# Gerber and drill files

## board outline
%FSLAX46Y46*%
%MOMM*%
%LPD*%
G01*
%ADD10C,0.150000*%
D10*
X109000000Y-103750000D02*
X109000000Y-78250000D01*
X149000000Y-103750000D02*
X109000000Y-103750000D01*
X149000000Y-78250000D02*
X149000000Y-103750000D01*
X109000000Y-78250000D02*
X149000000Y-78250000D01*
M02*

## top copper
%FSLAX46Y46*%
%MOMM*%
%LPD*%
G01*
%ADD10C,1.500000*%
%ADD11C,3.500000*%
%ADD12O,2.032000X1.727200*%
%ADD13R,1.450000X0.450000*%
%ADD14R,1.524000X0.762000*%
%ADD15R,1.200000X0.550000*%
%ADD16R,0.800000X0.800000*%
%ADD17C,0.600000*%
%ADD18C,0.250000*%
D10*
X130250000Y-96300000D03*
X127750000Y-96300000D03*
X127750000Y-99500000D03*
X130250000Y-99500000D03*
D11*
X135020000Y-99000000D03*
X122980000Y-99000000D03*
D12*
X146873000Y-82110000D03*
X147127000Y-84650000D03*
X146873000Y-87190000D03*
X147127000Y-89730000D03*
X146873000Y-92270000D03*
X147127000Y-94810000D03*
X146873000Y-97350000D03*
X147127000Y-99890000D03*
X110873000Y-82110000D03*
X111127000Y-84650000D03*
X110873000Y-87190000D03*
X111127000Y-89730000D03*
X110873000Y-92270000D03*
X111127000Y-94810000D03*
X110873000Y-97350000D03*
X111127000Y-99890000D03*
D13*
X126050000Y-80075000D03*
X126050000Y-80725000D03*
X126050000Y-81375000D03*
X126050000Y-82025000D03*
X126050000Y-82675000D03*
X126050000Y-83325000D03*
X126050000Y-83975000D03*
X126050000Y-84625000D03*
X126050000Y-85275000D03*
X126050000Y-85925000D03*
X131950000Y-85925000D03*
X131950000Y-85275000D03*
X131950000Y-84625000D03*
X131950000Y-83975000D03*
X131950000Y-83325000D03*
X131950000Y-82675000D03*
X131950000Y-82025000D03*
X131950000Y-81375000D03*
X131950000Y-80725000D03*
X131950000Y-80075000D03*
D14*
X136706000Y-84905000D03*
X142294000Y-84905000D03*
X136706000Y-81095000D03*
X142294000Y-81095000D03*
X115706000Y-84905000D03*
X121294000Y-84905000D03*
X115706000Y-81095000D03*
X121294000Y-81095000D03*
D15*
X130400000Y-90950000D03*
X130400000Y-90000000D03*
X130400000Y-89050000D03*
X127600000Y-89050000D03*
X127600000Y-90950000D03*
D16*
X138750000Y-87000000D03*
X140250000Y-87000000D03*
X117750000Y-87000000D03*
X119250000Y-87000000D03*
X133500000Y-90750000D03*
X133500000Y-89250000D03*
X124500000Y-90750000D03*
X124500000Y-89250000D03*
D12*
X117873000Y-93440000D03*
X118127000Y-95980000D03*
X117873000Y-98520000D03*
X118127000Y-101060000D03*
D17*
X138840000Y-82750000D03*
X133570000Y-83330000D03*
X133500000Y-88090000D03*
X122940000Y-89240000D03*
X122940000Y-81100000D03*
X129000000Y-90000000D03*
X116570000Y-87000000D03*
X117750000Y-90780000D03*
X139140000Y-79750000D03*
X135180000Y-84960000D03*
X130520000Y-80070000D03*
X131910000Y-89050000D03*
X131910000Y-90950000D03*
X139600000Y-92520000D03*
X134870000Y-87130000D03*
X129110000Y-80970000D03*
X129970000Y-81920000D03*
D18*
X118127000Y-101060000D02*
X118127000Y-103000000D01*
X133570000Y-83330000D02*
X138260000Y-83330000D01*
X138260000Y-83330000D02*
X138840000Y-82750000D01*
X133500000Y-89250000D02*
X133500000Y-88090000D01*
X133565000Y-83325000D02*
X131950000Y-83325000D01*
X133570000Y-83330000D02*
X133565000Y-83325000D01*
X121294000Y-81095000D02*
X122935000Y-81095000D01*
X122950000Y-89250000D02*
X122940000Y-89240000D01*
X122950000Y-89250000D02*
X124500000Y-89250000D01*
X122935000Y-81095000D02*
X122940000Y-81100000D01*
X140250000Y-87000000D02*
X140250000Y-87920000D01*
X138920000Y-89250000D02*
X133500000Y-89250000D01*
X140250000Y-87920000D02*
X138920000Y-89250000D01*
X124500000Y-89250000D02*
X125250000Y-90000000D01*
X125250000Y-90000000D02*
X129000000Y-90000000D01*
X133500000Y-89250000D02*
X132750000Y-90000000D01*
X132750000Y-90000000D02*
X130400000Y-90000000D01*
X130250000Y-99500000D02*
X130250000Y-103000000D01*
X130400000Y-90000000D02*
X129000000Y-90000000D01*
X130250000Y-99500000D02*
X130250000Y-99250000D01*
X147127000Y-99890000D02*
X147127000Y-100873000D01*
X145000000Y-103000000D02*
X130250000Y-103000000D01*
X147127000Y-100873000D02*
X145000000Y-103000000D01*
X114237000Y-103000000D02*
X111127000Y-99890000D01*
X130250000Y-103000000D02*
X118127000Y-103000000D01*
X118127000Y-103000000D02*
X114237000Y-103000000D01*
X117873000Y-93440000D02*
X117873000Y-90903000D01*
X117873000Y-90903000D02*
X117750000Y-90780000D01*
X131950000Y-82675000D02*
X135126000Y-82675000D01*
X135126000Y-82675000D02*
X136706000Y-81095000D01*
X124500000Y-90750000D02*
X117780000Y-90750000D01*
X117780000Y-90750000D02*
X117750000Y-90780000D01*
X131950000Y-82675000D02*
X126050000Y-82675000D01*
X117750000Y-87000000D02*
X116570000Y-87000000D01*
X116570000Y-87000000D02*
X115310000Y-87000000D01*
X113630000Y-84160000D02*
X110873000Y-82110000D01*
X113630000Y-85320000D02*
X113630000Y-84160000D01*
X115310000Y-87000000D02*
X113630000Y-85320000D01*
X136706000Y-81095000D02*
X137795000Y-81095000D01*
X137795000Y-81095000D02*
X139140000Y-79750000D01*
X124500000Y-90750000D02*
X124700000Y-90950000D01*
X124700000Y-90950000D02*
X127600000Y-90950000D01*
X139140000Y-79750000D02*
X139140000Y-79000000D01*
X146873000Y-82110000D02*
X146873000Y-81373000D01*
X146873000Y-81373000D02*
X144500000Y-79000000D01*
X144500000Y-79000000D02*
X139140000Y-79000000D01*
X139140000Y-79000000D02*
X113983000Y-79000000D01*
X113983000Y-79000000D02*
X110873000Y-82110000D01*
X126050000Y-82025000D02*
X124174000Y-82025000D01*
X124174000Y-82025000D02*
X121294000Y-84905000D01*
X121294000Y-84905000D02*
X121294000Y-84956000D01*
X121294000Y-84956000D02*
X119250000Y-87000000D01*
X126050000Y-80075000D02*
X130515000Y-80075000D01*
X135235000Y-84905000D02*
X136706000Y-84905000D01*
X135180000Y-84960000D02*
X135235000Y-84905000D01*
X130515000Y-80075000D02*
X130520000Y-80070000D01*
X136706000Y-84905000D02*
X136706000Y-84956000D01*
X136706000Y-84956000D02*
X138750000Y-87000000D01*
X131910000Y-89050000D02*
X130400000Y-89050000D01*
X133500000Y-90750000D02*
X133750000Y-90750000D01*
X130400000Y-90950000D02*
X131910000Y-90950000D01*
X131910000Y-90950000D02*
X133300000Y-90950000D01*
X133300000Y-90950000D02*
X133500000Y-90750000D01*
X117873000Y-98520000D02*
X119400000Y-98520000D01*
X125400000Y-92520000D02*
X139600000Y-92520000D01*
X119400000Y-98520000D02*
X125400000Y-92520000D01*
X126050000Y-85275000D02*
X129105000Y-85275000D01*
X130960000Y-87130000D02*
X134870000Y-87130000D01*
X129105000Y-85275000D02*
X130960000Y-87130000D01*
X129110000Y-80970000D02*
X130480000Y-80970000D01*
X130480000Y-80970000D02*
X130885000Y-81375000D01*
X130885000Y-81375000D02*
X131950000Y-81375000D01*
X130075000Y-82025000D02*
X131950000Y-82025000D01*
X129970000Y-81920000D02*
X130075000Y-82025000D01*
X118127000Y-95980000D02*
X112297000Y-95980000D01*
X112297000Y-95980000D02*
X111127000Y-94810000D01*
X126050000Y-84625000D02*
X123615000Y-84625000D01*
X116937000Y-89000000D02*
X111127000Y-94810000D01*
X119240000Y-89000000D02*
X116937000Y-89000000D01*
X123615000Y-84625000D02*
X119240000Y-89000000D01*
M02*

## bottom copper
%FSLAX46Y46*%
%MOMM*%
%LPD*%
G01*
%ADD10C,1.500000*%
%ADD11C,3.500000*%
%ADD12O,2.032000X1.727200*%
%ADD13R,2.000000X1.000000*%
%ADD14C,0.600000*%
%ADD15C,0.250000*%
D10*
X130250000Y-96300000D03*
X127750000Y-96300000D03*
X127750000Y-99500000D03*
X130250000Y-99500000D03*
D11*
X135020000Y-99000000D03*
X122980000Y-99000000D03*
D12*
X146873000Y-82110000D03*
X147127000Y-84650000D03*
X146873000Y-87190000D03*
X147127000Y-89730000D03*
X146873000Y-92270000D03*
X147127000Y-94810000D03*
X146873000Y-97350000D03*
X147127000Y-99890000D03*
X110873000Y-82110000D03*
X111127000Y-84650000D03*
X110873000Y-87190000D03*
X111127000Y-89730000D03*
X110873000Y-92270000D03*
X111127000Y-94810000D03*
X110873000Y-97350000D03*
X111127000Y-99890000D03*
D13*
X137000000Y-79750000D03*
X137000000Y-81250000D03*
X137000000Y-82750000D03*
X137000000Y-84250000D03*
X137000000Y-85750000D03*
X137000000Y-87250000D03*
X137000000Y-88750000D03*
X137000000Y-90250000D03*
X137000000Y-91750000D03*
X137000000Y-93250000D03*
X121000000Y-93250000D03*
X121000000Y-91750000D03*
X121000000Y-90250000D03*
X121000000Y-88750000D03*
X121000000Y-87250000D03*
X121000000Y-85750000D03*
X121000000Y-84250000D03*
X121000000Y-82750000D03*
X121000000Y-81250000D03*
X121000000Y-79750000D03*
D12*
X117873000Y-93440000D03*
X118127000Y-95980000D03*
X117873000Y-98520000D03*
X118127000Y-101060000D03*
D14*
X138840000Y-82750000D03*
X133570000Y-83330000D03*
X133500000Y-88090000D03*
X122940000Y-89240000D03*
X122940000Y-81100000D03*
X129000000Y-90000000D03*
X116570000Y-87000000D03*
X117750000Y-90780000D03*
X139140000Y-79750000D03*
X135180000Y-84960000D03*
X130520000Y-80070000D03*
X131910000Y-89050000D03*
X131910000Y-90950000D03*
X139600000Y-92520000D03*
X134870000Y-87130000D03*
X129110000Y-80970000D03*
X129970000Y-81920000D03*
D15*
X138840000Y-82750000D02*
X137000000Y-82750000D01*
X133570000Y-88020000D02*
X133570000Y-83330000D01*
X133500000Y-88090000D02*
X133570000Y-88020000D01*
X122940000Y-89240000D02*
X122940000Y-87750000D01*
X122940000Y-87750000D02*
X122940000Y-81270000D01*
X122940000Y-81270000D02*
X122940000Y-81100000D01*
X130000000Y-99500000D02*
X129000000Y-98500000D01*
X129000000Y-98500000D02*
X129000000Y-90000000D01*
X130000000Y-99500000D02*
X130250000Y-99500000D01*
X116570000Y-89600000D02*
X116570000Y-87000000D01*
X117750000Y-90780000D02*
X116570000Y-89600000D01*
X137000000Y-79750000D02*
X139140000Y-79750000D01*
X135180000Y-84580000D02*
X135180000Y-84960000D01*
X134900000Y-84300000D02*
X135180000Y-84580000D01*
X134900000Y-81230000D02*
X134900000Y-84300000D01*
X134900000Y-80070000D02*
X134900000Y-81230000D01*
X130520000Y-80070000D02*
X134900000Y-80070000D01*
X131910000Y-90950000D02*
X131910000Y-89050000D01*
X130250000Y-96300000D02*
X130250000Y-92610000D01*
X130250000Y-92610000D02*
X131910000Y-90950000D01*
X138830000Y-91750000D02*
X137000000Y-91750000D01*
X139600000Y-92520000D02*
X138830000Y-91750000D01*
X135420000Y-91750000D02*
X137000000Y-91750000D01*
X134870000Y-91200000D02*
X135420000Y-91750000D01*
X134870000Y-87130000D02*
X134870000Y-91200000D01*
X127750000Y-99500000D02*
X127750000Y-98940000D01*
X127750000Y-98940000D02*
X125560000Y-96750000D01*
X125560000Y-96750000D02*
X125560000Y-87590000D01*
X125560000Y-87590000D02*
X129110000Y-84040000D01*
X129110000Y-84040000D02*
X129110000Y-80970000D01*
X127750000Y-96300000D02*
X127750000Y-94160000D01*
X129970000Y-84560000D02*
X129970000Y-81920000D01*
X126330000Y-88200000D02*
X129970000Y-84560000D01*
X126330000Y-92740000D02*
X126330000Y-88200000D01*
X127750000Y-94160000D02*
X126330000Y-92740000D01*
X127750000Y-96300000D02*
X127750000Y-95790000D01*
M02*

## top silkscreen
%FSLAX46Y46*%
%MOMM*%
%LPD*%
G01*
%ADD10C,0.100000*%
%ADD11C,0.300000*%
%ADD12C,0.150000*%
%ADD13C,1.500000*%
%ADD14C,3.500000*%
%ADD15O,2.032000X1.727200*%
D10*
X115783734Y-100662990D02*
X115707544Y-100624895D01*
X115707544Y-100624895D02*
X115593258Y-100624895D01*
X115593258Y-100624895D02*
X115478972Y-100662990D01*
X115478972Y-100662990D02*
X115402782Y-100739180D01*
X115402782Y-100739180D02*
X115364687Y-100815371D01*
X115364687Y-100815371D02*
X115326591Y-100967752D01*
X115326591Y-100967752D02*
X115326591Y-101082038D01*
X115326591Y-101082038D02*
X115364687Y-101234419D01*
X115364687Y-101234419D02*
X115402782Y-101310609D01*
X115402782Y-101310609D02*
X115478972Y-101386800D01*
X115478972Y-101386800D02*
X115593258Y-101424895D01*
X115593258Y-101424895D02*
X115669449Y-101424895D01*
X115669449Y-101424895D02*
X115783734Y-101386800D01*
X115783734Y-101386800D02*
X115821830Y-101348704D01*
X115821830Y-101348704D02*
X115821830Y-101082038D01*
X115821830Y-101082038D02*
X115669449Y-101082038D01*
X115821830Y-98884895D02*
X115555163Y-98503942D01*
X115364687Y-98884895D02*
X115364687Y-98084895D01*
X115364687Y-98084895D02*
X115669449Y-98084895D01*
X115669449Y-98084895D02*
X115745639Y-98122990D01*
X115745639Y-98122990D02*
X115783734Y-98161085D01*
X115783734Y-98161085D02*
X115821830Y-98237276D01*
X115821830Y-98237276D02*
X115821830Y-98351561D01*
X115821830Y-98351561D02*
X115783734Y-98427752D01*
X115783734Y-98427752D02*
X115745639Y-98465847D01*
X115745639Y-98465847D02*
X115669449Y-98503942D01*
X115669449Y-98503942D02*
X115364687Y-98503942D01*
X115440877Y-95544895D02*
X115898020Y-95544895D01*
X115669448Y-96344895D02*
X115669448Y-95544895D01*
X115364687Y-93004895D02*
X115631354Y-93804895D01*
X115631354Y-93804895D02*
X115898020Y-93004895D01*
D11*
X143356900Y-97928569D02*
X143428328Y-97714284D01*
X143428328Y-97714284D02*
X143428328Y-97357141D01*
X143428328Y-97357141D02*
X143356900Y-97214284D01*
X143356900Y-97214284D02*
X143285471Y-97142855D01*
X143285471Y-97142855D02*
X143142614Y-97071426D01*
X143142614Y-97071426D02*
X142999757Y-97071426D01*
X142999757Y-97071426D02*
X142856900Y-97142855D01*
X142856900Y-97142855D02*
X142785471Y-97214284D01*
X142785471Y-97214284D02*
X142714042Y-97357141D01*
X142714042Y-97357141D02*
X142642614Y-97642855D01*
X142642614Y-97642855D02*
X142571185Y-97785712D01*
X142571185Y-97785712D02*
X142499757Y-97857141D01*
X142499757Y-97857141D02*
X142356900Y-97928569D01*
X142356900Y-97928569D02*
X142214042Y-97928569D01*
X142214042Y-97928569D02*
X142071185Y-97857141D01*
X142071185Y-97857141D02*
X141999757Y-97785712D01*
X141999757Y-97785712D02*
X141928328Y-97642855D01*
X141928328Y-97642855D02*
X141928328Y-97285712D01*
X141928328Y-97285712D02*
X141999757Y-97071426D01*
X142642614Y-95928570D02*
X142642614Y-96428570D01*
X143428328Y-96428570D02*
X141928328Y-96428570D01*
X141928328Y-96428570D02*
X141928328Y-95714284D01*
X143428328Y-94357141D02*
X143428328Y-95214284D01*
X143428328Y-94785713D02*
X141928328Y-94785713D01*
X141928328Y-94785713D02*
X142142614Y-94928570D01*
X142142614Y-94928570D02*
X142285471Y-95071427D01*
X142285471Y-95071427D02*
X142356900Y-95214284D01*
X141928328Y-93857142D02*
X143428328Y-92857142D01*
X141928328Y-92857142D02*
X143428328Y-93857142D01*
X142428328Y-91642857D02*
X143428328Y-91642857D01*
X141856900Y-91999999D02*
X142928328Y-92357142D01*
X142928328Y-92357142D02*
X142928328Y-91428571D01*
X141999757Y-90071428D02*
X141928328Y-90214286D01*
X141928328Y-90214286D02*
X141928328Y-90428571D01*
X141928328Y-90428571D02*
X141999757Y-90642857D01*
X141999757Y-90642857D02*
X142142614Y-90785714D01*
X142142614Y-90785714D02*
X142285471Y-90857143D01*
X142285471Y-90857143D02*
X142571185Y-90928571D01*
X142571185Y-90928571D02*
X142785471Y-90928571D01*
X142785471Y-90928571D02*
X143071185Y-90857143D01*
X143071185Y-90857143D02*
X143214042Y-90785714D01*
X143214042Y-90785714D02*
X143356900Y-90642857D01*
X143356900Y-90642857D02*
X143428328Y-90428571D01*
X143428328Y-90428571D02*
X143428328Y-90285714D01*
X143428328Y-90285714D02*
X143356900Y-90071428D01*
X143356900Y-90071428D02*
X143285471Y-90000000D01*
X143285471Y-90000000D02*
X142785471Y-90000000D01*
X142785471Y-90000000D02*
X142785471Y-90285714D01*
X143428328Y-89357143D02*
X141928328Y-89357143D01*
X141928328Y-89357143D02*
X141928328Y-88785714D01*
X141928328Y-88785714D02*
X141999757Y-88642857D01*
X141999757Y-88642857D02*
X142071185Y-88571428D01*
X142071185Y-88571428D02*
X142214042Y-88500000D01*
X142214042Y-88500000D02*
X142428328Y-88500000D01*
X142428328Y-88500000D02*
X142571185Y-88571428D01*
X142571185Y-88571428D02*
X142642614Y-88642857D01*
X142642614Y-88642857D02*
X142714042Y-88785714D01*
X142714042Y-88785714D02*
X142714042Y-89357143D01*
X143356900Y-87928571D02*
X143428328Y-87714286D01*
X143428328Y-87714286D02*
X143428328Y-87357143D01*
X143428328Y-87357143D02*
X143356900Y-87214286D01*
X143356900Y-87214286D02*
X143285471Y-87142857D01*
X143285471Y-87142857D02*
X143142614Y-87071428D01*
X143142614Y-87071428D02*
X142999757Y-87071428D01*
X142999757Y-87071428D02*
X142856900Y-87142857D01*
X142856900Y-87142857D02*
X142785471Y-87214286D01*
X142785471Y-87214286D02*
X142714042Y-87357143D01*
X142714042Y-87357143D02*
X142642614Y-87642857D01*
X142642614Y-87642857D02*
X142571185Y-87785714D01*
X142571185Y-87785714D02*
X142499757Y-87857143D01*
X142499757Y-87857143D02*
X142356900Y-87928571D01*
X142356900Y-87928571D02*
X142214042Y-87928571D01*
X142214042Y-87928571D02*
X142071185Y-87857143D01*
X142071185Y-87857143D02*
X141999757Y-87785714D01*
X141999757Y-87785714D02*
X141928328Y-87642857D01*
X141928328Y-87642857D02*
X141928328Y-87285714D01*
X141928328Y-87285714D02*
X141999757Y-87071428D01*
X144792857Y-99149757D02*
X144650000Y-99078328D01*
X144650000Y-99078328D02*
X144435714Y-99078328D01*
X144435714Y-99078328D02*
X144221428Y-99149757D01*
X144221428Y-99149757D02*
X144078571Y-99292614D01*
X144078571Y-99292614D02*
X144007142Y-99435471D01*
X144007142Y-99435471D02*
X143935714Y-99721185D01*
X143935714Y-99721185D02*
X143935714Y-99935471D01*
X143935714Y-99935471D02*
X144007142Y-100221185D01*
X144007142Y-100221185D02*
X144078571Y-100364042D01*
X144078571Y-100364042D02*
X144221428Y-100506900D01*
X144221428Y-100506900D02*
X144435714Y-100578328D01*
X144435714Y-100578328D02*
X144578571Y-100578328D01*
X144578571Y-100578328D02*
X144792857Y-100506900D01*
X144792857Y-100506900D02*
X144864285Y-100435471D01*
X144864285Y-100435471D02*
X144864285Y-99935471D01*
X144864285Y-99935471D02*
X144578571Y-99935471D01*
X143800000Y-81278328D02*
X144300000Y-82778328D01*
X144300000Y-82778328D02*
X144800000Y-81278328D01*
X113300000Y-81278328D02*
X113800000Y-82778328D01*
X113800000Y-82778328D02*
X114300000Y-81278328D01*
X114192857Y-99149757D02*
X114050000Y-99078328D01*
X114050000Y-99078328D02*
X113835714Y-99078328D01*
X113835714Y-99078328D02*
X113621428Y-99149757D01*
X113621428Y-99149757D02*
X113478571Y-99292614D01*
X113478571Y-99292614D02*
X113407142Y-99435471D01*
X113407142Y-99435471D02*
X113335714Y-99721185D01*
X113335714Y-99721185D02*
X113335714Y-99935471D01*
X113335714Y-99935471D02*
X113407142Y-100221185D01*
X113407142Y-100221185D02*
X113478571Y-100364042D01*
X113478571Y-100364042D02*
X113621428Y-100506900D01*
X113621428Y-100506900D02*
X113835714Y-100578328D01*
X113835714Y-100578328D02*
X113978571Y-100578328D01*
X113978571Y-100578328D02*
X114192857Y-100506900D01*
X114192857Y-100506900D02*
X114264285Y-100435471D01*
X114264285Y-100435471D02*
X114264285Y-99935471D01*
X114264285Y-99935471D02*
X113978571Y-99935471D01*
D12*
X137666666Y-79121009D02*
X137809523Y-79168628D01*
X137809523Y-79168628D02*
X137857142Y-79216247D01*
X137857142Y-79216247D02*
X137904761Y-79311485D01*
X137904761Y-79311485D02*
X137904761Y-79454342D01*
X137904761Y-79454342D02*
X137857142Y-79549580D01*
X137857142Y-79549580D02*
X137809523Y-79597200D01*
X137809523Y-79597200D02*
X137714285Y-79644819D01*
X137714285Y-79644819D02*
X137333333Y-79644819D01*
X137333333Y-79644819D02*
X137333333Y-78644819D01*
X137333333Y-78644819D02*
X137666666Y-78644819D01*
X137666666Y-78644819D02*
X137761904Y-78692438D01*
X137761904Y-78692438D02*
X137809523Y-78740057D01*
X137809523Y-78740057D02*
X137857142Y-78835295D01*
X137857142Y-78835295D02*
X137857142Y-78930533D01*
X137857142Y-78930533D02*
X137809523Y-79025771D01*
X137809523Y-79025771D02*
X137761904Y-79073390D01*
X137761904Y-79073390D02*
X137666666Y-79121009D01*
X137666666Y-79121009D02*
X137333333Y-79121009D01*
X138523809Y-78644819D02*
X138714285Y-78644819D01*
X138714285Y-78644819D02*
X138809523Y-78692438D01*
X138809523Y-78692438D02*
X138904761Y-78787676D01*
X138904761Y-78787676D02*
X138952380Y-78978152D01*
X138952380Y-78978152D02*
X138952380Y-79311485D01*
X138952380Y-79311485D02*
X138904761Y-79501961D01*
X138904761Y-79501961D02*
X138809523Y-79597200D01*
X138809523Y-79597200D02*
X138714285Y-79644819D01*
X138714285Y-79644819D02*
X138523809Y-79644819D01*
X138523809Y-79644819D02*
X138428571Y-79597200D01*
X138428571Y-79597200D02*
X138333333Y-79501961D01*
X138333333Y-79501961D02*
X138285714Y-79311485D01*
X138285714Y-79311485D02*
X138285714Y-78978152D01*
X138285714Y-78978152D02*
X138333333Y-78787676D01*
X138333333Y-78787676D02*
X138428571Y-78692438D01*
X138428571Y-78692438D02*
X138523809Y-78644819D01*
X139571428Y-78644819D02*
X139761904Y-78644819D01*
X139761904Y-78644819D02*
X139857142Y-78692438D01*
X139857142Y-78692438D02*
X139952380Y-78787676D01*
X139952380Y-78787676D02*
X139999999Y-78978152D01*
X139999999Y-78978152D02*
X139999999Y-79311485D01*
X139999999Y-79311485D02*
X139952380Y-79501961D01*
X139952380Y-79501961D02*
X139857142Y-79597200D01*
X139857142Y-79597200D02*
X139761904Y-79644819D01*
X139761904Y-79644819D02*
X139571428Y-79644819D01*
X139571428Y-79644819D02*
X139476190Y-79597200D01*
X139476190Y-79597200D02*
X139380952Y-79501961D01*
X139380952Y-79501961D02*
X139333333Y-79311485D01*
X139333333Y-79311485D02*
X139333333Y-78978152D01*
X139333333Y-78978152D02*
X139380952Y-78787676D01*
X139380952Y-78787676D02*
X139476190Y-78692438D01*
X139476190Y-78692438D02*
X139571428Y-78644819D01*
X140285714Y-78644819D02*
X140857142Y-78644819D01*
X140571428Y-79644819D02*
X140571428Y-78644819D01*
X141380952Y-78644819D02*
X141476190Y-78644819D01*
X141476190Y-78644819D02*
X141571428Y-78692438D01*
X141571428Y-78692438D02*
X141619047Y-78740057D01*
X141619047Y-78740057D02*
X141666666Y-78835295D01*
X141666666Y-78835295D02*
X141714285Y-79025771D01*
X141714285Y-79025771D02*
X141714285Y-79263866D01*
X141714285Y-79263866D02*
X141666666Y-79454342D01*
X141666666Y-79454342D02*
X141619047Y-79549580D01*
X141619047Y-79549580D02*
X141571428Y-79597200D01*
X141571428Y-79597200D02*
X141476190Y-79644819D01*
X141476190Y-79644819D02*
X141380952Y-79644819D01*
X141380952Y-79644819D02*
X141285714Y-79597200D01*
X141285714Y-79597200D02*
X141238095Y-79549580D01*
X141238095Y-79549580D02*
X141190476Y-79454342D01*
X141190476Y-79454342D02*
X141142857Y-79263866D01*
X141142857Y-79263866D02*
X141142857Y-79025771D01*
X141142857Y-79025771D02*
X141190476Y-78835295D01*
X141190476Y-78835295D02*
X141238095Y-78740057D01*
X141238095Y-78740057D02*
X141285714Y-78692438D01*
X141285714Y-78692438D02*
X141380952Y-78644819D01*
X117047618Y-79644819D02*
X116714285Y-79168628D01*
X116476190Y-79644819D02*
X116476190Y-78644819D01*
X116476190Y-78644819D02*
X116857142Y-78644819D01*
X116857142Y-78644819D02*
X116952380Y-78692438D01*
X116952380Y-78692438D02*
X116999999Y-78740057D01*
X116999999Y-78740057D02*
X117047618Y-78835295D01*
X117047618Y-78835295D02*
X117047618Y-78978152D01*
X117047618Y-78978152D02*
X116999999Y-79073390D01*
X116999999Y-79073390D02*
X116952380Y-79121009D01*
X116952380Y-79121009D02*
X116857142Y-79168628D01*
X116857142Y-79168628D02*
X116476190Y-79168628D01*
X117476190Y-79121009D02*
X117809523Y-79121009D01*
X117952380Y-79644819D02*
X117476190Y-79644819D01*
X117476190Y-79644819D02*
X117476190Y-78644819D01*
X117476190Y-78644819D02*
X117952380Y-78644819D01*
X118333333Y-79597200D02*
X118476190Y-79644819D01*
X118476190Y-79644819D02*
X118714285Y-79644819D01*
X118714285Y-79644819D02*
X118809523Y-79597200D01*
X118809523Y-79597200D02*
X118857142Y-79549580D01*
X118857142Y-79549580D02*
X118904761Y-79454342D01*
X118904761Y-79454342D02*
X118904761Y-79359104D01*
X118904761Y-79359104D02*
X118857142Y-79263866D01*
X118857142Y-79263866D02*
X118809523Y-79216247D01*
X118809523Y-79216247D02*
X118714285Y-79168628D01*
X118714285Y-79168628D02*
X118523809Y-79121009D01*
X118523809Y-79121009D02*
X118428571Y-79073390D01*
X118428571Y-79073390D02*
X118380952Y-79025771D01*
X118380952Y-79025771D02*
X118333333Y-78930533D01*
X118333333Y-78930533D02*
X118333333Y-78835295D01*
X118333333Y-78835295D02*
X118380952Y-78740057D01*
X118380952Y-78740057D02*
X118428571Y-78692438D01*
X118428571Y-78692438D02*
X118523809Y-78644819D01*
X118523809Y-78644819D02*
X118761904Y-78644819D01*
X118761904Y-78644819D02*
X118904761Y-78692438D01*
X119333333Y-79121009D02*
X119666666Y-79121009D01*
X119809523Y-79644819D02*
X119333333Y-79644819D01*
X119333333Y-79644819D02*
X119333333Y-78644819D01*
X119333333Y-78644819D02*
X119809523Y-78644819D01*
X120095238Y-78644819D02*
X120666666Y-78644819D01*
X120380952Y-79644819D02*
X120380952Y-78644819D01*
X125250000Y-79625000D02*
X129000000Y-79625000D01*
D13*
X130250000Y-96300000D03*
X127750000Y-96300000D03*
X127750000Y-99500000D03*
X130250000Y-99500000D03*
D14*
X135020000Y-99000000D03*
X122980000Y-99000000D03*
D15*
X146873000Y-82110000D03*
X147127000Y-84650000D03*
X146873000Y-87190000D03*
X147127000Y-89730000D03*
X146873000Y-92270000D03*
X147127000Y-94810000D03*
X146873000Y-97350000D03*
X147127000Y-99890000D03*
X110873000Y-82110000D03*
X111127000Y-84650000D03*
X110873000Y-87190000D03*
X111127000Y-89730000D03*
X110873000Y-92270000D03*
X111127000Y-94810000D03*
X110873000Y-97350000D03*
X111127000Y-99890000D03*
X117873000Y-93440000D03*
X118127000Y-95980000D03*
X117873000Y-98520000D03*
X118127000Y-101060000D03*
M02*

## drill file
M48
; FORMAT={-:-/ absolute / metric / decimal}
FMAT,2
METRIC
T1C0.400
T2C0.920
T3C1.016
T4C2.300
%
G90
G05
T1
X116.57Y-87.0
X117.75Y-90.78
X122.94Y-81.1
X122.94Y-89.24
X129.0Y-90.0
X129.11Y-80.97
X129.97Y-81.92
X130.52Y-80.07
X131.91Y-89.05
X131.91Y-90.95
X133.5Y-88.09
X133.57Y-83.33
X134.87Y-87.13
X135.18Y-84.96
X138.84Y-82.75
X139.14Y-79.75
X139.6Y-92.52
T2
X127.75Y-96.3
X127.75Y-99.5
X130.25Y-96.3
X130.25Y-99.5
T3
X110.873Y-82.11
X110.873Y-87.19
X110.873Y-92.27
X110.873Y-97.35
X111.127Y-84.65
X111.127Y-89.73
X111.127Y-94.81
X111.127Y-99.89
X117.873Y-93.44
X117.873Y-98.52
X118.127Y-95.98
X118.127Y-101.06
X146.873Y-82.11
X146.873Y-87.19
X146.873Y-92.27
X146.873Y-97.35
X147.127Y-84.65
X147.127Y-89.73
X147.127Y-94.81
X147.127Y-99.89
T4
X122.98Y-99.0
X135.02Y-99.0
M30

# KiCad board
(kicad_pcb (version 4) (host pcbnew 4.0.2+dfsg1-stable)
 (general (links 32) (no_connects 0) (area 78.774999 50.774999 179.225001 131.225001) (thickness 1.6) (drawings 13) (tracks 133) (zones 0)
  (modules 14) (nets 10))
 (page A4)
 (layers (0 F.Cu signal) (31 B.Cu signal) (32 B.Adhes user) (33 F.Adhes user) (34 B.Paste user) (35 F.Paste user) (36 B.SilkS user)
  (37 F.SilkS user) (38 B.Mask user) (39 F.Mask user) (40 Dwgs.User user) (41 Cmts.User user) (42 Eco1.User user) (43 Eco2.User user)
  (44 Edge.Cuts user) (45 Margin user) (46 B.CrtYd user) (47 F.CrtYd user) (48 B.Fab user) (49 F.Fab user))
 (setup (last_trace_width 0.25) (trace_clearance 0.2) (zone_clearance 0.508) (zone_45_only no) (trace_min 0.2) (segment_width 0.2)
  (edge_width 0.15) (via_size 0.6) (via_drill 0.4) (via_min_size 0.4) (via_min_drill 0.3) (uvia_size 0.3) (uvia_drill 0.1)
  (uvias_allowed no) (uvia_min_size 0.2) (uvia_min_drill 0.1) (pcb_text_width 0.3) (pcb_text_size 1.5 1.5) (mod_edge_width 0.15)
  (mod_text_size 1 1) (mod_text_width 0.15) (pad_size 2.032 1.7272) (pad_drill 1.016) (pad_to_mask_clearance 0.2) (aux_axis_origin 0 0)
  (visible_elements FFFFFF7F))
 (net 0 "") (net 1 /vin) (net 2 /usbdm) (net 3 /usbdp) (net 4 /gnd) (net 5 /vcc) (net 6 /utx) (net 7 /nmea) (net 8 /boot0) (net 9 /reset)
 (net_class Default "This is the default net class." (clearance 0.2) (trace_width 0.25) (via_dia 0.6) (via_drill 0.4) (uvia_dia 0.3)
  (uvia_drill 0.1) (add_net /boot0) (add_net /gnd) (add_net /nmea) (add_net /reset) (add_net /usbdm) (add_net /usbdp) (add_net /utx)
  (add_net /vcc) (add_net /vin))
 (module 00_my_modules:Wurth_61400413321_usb (layer F.Cu) (at 129 99)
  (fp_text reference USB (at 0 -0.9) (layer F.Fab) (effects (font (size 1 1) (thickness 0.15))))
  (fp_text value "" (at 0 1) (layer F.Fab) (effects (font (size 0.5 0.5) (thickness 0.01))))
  (pad V thru_hole circle (at 1.25 -2.7) (size 1.5 1.5) (drill 0.92) (layers *.Cu *.Mask F.SilkS) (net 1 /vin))
  (pad - thru_hole circle (at -1.25 -2.7) (size 1.5 1.5) (drill 0.92) (layers *.Cu *.Mask F.SilkS) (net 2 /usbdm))
  (pad + thru_hole circle (at -1.25 0.5) (size 1.5 1.5) (drill 0.92) (layers *.Cu *.Mask F.SilkS) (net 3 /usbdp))
  (pad G thru_hole circle (at 1.25 0.5) (size 1.5 1.5) (drill 0.92) (layers *.Cu *.Mask F.SilkS) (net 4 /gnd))
  (pad X thru_hole circle (at 6.02 0) (size 3.5 3.5) (drill 2.3) (layers *.Cu *.Mask F.SilkS))
  (pad X thru_hole circle (at -6.02 0) (size 3.5 3.5) (drill 2.3) (layers *.Cu *.Mask F.SilkS)))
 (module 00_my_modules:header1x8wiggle (layer F.Cu) (at 147 91)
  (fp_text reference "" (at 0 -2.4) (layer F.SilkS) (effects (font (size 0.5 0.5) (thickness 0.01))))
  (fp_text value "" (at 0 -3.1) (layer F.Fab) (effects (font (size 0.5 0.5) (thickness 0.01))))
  (pad 1 thru_hole oval (at -0.127 -8.89) (size 2.032 1.7272) (drill 1.016) (layers *.Cu *.Mask F.SilkS) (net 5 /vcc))
  (pad 2 thru_hole oval (at 0.127 -6.35) (size 2.032 1.7272) (drill 1.016) (layers *.Cu *.Mask F.SilkS))
  (pad 3 thru_hole oval (at -0.127 -3.81) (size 2.032 1.7272) (drill 1.016) (layers *.Cu *.Mask F.SilkS))
  (pad 4 thru_hole oval (at 0.127 -1.27) (size 2.032 1.7272) (drill 1.016) (layers *.Cu *.Mask F.SilkS))
  (pad 5 thru_hole oval (at -0.127 1.27) (size 2.032 1.7272) (drill 1.016) (layers *.Cu *.Mask F.SilkS))
  (pad 6 thru_hole oval (at 0.127 3.81) (size 2.032 1.7272) (drill 1.016) (layers *.Cu *.Mask F.SilkS))
  (pad 7 thru_hole oval (at -0.127 6.35) (size 2.032 1.7272) (drill 1.016) (layers *.Cu *.Mask F.SilkS))
  (pad 8 thru_hole oval (at 0.127 8.89) (size 2.032 1.7272) (drill 1.016) (layers *.Cu *.Mask F.SilkS) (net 4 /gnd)))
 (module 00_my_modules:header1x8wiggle (layer F.Cu) (at 111 91)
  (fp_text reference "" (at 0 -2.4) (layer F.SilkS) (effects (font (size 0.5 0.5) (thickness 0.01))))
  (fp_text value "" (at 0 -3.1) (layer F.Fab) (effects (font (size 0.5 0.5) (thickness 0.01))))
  (pad 1 thru_hole oval (at -0.127 -8.89) (size 2.032 1.7272) (drill 1.016) (layers *.Cu *.Mask F.SilkS) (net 5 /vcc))
  (pad 2 thru_hole oval (at 0.127 -6.35) (size 2.032 1.7272) (drill 1.016) (layers *.Cu *.Mask F.SilkS))
  (pad 3 thru_hole oval (at -0.127 -3.81) (size 2.032 1.7272) (drill 1.016) (layers *.Cu *.Mask F.SilkS))
  (pad 4 thru_hole oval (at 0.127 -1.27) (size 2.032 1.7272) (drill 1.016) (layers *.Cu *.Mask F.SilkS))
  (pad 5 thru_hole oval (at -0.127 1.27) (size 2.032 1.7272) (drill 1.016) (layers *.Cu *.Mask F.SilkS))
  (pad 6 thru_hole oval (at 0.127 3.81) (size 2.032 1.7272) (drill 1.016) (layers *.Cu *.Mask F.SilkS) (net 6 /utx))
  (pad 7 thru_hole oval (at -0.127 6.35) (size 2.032 1.7272) (drill 1.016) (layers *.Cu *.Mask F.SilkS))
  (pad 8 thru_hole oval (at 0.127 8.89) (size 2.032 1.7272) (drill 1.016) (layers *.Cu *.Mask F.SilkS) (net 4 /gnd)))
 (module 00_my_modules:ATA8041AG (layer B.Cu) (at 129 91 180)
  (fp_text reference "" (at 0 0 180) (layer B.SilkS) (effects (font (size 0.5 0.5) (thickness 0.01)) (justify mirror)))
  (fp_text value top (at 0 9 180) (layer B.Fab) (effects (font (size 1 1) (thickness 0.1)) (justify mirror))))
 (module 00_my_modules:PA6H (layer B.Cu) (at 129 86.5 180)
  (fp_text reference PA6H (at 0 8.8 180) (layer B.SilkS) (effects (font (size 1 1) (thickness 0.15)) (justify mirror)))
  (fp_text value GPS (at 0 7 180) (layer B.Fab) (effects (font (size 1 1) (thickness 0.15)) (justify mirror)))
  (pad VCC smd rect (at -8 6.75 180) (size 2 1) (layers B.Cu B.Paste B.Mask) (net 5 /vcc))
  (pad 2 smd rect (at -8 5.25 180) (size 2 1) (layers B.Cu B.Paste B.Mask))
  (pad GND smd rect (at -8 3.75 180) (size 2 1) (layers B.Cu B.Paste B.Mask) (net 4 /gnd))
  (pad 4 smd rect (at -8 2.25 180) (size 2 1) (layers B.Cu B.Paste B.Mask))
  (pad 5 smd rect (at -8 0.75 180) (size 2 1) (layers B.Cu B.Paste B.Mask))
  (pad 6 smd rect (at -8 -0.75 180) (size 2 1) (layers B.Cu B.Paste B.Mask))
  (pad 7 smd rect (at -8 -2.25 180) (size 2 1) (layers B.Cu B.Paste B.Mask))
  (pad 8 smd rect (at -8 -3.75 180) (size 2 1) (layers B.Cu B.Paste B.Mask))
  (pad TX smd rect (at -8 -5.25 180) (size 2 1) (layers B.Cu B.Paste B.Mask) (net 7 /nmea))
  (pad RX smd rect (at -8 -6.75 180) (size 2 1) (layers B.Cu B.Paste B.Mask))
  (pad 11 smd rect (at 8 -6.75 180) (size 2 1) (layers B.Cu B.Paste B.Mask))
  (pad 12 smd rect (at 8 -5.25 180) (size 2 1) (layers B.Cu B.Paste B.Mask))
  (pad 13 smd rect (at 8 -3.75 180) (size 2 1) (layers B.Cu B.Paste B.Mask))
  (pad 14 smd rect (at 8 -2.25 180) (size 2 1) (layers B.Cu B.Paste B.Mask))
  (pad 15 smd rect (at 8 -0.75 180) (size 2 1) (layers B.Cu B.Paste B.Mask))
  (pad 16 smd rect (at 8 0.75 180) (size 2 1) (layers B.Cu B.Paste B.Mask))
  (pad 17 smd rect (at 8 2.25 180) (size 2 1) (layers B.Cu B.Paste B.Mask))
  (pad 18 smd rect (at 8 3.75 180) (size 2 1) (layers B.Cu B.Paste B.Mask))
  (pad 19 smd rect (at 8 5.25 180) (size 2 1) (layers B.Cu B.Paste B.Mask))
  (pad 20 smd rect (at 8 6.75 180) (size 2 1) (layers B.Cu B.Paste B.Mask)))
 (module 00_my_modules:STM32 (layer F.Cu) (at 129 83)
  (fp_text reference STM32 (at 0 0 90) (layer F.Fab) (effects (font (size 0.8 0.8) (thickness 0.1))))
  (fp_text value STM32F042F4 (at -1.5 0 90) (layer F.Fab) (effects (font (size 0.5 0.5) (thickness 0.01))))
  (fp_line (start -3.75 -3.375) (end 0 -3.375) (layer F.SilkS) (width 0.15))
  (pad BOOT smd rect (at -2.95 -2.925) (size 1.45 0.45) (layers F.Cu F.Paste F.Mask) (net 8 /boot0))
  (pad 2 smd rect (at -2.95 -2.275) (size 1.45 0.45) (layers F.Cu F.Paste F.Mask))
  (pad 3 smd rect (at -2.95 -1.625) (size 1.45 0.45) (layers F.Cu F.Paste F.Mask))
  (pad NRST smd rect (at -2.95 -0.975) (size 1.45 0.45) (layers F.Cu F.Paste F.Mask) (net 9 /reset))
  (pad VCC smd rect (at -2.95 -0.325) (size 1.45 0.45) (layers F.Cu F.Paste F.Mask) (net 5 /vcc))
  (pad PA0 smd rect (at -2.95 0.325) (size 1.45 0.45) (layers F.Cu F.Paste F.Mask))
  (pad PA1 smd rect (at -2.95 0.975) (size 1.45 0.45) (layers F.Cu F.Paste F.Mask))
  (pad PA2 smd rect (at -2.95 1.625) (size 1.45 0.45) (layers F.Cu F.Paste F.Mask) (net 6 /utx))
  (pad PA3 smd rect (at -2.95 2.275) (size 1.45 0.45) (layers F.Cu F.Paste F.Mask) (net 7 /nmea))
  (pad PA4 smd rect (at -2.95 2.925) (size 1.45 0.45) (layers F.Cu F.Paste F.Mask))
  (pad PA5 smd rect (at 2.95 2.925) (size 1.45 0.45) (layers F.Cu F.Paste F.Mask))
  (pad PA6 smd rect (at 2.95 2.275) (size 1.45 0.45) (layers F.Cu F.Paste F.Mask))
  (pad PA7 smd rect (at 2.95 1.625) (size 1.45 0.45) (layers F.Cu F.Paste F.Mask))
  (pad PB1 smd rect (at 2.95 0.975) (size 1.45 0.45) (layers F.Cu F.Paste F.Mask))
  (pad GND smd rect (at 2.95 0.325) (size 1.45 0.45) (layers F.Cu F.Paste F.Mask) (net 4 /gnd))
  (pad VCC smd rect (at 2.95 -0.325) (size 1.45 0.45) (layers F.Cu F.Paste F.Mask) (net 5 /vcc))
  (pad PA11 smd rect (at 2.95 -0.975) (size 1.45 0.45) (layers F.Cu F.Paste F.Mask) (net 2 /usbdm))
  (pad PA12 smd rect (at 2.95 -1.625) (size 1.45 0.45) (layers F.Cu F.Paste F.Mask) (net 3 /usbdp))
  (pad PA13 smd rect (at 2.95 -2.275) (size 1.45 0.45) (layers F.Cu F.Paste F.Mask))
  (pad PA14 smd rect (at 2.95 -2.925) (size 1.45 0.45) (layers F.Cu F.Paste F.Mask)))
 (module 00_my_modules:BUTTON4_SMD (layer F.Cu) (at 139.5 83)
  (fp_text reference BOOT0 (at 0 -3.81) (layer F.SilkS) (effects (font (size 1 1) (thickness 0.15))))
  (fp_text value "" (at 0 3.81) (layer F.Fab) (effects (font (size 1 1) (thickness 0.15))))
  (pad 1 smd rect (at -2.794 1.905) (size 1.524 0.762) (layers F.Cu F.Paste F.Mask) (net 8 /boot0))
  (pad 2 smd rect (at 2.794 1.905) (size 1.524 0.762) (layers F.Cu F.Paste F.Mask))
  (pad 3 smd rect (at -2.794 -1.905) (size 1.524 0.762) (layers F.Cu F.Paste F.Mask) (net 5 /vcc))
  (pad 4 smd rect (at 2.794 -1.905) (size 1.524 0.762) (layers F.Cu F.Paste F.Mask)))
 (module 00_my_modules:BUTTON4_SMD (layer F.Cu) (at 118.5 83)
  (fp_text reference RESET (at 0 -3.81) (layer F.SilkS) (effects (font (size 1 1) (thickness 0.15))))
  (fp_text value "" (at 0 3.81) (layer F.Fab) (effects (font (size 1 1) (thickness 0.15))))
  (pad 1 smd rect (at -2.794 1.905) (size 1.524 0.762) (layers F.Cu F.Paste F.Mask))
  (pad 2 smd rect (at 2.794 1.905) (size 1.524 0.762) (layers F.Cu F.Paste F.Mask) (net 9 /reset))
  (pad 3 smd rect (at -2.794 -1.905) (size 1.524 0.762) (layers F.Cu F.Paste F.Mask))
  (pad 4 smd rect (at 2.794 -1.905) (size 1.524 0.762) (layers F.Cu F.Paste F.Mask) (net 4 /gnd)))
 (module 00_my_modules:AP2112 (layer F.Cu) (at 129 90 180)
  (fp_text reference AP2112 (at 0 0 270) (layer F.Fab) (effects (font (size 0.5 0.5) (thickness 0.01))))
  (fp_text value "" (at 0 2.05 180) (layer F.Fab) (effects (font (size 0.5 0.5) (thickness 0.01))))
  (pad VIN smd rect (at -1.4 -0.95 180) (size 1.2 0.55) (layers F.Cu F.Paste F.Mask) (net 1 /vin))
  (pad GND smd rect (at -1.4 0 180) (size 1.2 0.55) (layers F.Cu F.Paste F.Mask) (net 4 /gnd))
  (pad EN smd rect (at -1.4 0.95 180) (size 1.2 0.55) (layers F.Cu F.Paste F.Mask) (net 1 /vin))
  (pad NC smd rect (at 1.4 0.95 180) (size 1.2 0.55) (layers F.Cu F.Paste F.Mask))
  (pad VOUT smd rect (at 1.4 -0.95 180) (size 1.2 0.55) (layers F.Cu F.Paste F.Mask) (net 5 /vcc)))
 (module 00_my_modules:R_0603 (layer F.Cu) (at 139.5 87)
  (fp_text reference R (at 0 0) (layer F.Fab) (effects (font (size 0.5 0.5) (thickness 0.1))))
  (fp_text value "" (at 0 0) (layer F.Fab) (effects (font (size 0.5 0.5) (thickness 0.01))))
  (pad 1 smd rect (at -0.75 0) (size 0.8 0.8) (layers F.Cu F.Paste F.Mask) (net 8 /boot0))
  (pad 2 smd rect (at 0.75 0) (size 0.8 0.8) (layers F.Cu F.Paste F.Mask) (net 4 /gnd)))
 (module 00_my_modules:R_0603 (layer F.Cu) (at 118.5 87)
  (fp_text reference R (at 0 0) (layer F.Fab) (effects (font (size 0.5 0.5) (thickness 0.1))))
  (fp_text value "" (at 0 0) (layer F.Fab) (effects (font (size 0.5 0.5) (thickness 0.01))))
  (pad 1 smd rect (at -0.75 0) (size 0.8 0.8) (layers F.Cu F.Paste F.Mask) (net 5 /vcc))
  (pad 2 smd rect (at 0.75 0) (size 0.8 0.8) (layers F.Cu F.Paste F.Mask) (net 9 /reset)))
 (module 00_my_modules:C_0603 (layer F.Cu) (at 133.5 90 90)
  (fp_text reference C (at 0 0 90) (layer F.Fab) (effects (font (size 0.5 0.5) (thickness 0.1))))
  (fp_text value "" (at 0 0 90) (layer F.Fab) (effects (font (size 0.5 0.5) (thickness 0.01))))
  (pad 1 smd rect (at -0.75 0 90) (size 0.8 0.8) (layers F.Cu F.Paste F.Mask) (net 1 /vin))
  (pad 2 smd rect (at 0.75 0 90) (size 0.8 0.8) (layers F.Cu F.Paste F.Mask) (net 4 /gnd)))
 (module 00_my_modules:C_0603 (layer F.Cu) (at 124.5 90 90)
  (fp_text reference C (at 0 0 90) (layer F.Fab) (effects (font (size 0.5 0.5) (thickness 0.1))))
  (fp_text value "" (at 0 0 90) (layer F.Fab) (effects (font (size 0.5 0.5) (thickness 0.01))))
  (pad 1 smd rect (at -0.75 0 90) (size 0.8 0.8) (layers F.Cu F.Paste F.Mask) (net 5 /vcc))
  (pad 2 smd rect (at 0.75 0 90) (size 0.8 0.8) (layers F.Cu F.Paste F.Mask) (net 4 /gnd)))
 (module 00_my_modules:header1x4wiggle (layer F.Cu) (at 118 97.25)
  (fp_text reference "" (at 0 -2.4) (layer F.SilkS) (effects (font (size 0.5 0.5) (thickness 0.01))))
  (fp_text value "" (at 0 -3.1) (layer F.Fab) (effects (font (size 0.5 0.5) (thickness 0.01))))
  (pad 1 thru_hole oval (at -0.127 -3.81) (size 2.032 1.7272) (drill 1.016) (layers *.Cu *.Mask F.SilkS) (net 5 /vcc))
  (pad 2 thru_hole oval (at 0.127 -1.27) (size 2.032 1.7272) (drill 1.016) (layers *.Cu *.Mask F.SilkS) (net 6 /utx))
  (pad 3 thru_hole oval (at -0.127 1.27) (size 2.032 1.7272) (drill 1.016) (layers *.Cu *.Mask F.SilkS) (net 7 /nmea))
  (pad 4 thru_hole oval (at 0.127 3.81) (size 2.032 1.7272) (drill 1.016) (layers *.Cu *.Mask F.SilkS) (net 4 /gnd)))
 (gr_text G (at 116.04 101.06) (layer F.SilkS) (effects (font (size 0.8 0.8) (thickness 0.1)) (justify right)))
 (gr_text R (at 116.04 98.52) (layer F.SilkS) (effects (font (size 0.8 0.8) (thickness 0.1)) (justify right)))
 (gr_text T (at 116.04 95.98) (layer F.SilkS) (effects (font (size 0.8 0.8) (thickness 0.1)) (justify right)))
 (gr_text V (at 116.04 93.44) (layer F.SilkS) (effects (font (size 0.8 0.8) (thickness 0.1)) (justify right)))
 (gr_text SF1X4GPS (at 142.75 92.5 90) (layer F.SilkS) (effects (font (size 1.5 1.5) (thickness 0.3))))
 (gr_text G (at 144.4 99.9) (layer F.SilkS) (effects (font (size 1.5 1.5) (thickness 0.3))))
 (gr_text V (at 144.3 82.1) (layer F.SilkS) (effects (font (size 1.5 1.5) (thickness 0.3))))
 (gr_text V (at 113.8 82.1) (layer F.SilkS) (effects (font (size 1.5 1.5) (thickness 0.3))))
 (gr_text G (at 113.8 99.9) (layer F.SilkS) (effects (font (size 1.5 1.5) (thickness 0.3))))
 (gr_line (start 109 103.75) (end 109 78.25) (angle 90) (layer Edge.Cuts) (width 0.15))
 (gr_line (start 149 103.75) (end 109 103.75) (angle 90) (layer Edge.Cuts) (width 0.15))
 (gr_line (start 149 78.25) (end 149 103.75) (angle 90) (layer Edge.Cuts) (width 0.15))
 (gr_line (start 109 78.25) (end 149 78.25) (angle 90) (layer Edge.Cuts) (width 0.15))
 (segment (start 118.127 101.06) (end 118.127 103) (width 0.25) (layer F.Cu) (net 4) (status 400000))
 (segment (start 133.57 83.33) (end 138.26 83.33) (width 0.25) (layer F.Cu) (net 4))
 (segment (start 138.84 82.75) (end 137 82.75) (width 0.25) (layer B.Cu) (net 4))
 (via (at 138.84 82.75) (size 0.6) (drill 0.4) (layers F.Cu B.Cu) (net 4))
 (segment (start 138.26 83.33) (end 138.84 82.75) (width 0.25) (layer F.Cu) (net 4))
 (segment (start 133.5 89.25) (end 133.5 88.09) (width 0.25) (layer F.Cu) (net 4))
 (segment (start 133.565 83.325) (end 131.95 83.325) (width 0.25) (layer F.Cu) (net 4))
 (segment (start 133.57 83.33) (end 133.565 83.325) (width 0.25) (layer F.Cu) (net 4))
 (via (at 133.57 83.33) (size 0.6) (drill 0.4) (layers F.Cu B.Cu) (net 4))
 (segment (start 133.57 88.02) (end 133.57 83.33) (width 0.25) (layer B.Cu) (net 4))
 (segment (start 133.5 88.09) (end 133.57 88.02) (width 0.25) (layer B.Cu) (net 4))
 (via (at 133.5 88.09) (size 0.6) (drill 0.4) (layers F.Cu B.Cu) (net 4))
 (segment (start 121.294 81.095) (end 122.935 81.095) (width 0.25) (layer F.Cu) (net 4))
 (segment (start 122.95 89.25) (end 122.94 89.24) (width 0.25) (layer F.Cu) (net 4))
 (via (at 122.94 89.24) (size 0.6) (drill 0.4) (layers F.Cu B.Cu) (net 4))
 (segment (start 122.94 89.24) (end 122.94 87.75) (width 0.25) (layer B.Cu) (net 4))
 (segment (start 122.94 87.75) (end 122.94 81.27) (width 0.25) (layer B.Cu) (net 4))
 (segment (start 122.94 81.27) (end 122.94 81.1) (width 0.25) (layer B.Cu) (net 4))
 (via (at 122.94 81.1) (size 0.6) (drill 0.4) (layers F.Cu B.Cu) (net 4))
 (segment (start 122.95 89.25) (end 124.5 89.25) (width 0.25) (layer F.Cu) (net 4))
 (segment (start 122.935 81.095) (end 122.94 81.1) (width 0.25) (layer F.Cu) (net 4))
 (segment (start 140.25 87) (end 140.25 87.92) (width 0.25) (layer F.Cu) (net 4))
 (segment (start 138.92 89.25) (end 133.5 89.25) (width 0.25) (layer F.Cu) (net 4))
 (segment (start 140.25 87.92) (end 138.92 89.25) (width 0.25) (layer F.Cu) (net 4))
 (via (at 129 90) (size 0.6) (drill 0.4) (layers F.Cu B.Cu) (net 4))
 (segment (start 130 99.5) (end 129 98.5) (width 0.25) (layer B.Cu) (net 4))
 (segment (start 129 98.5) (end 129 90) (width 0.25) (layer B.Cu) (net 4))
 (segment (start 130 99.5) (end 130.25 99.5) (width 0.25) (layer B.Cu) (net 4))
 (segment (start 124.5 89.25) (end 125.25 90) (width 0.25) (layer F.Cu) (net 4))
 (segment (start 125.25 90) (end 129 90) (width 0.25) (layer F.Cu) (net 4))
 (segment (start 133.5 89.25) (end 132.75 90) (width 0.25) (layer F.Cu) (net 4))
 (segment (start 132.75 90) (end 130.4 90) (width 0.25) (layer F.Cu) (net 4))
 (segment (start 130.25 99.5) (end 130.25 103) (width 0.25) (layer F.Cu) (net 4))
 (segment (start 130.4 90) (end 129 90) (width 0.25) (layer F.Cu) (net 4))
 (segment (start 130.25 99.5) (end 130.25 99.25) (width 0.25) (layer F.Cu) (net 4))
 (segment (start 147.127 99.89) (end 147.127 100.873) (width 0.25) (layer F.Cu) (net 4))
 (segment (start 145 103) (end 130.25 103) (width 0.25) (layer F.Cu) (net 4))
 (segment (start 147.127 100.873) (end 145 103) (width 0.25) (layer F.Cu) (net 4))
 (segment (start 114.237 103) (end 111.127 99.89) (width 0.25) (layer F.Cu) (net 4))
 (segment (start 130.25 103) (end 118.127 103) (width 0.25) (layer F.Cu) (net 4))
 (segment (start 118.127 103) (end 114.237 103) (width 0.25) (layer F.Cu) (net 4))
 (segment (start 117.873 93.44) (end 117.873 90.903) (width 0.25) (layer F.Cu) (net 5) (status 400000))
 (segment (start 117.873 90.903) (end 117.75 90.78) (width 0.25) (layer F.Cu) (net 5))
 (segment (start 131.95 82.675) (end 135.126 82.675) (width 0.25) (layer F.Cu) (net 5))
 (segment (start 135.126 82.675) (end 136.706 81.095) (width 0.25) (layer F.Cu) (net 5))
 (segment (start 124.5 90.75) (end 117.78 90.75) (width 0.25) (layer F.Cu) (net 5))
 (via (at 116.57 87) (size 0.6) (drill 0.4) (layers F.Cu B.Cu) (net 5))
 (segment (start 116.57 89.6) (end 116.57 87) (width 0.25) (layer B.Cu) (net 5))
 (segment (start 117.75 90.78) (end 116.57 89.6) (width 0.25) (layer B.Cu) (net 5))
 (via (at 117.75 90.78) (size 0.6) (drill 0.4) (layers F.Cu B.Cu) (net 5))
 (segment (start 117.78 90.75) (end 117.75 90.78) (width 0.25) (layer F.Cu) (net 5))
 (segment (start 131.95 82.675) (end 126.05 82.675) (width 0.25) (layer F.Cu) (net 5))
 (segment (start 117.75 87) (end 116.57 87) (width 0.25) (layer F.Cu) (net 5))
 (segment (start 116.57 87) (end 115.31 87) (width 0.25) (layer F.Cu) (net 5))
 (segment (start 113.63 84.16) (end 110.873 82.11) (width 0.25) (layer F.Cu) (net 5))
 (segment (start 113.63 85.32) (end 113.63 84.16) (width 0.25) (layer F.Cu) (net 5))
 (segment (start 115.31 87) (end 113.63 85.32) (width 0.25) (layer F.Cu) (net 5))
 (segment (start 136.706 81.095) (end 137.795 81.095) (width 0.25) (layer F.Cu) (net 5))
 (segment (start 137.795 81.095) (end 139.14 79.75) (width 0.25) (layer F.Cu) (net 5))
 (segment (start 124.5 90.75) (end 124.7 90.95) (width 0.25) (layer F.Cu) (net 5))
 (segment (start 124.7 90.95) (end 127.6 90.95) (width 0.25) (layer F.Cu) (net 5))
 (segment (start 137 79.75) (end 139.14 79.75) (width 0.25) (layer B.Cu) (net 5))
 (segment (start 139.14 79.75) (end 139.14 79) (width 0.25) (layer F.Cu) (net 5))
 (via (at 139.14 79.75) (size 0.6) (drill 0.4) (layers F.Cu B.Cu) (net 5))
 (segment (start 146.873 82.11) (end 146.873 81.373) (width 0.25) (layer F.Cu) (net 5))
 (segment (start 146.873 81.373) (end 144.5 79) (width 0.25) (layer F.Cu) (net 5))
 (segment (start 144.5 79) (end 139.14 79) (width 0.25) (layer F.Cu) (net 5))
 (segment (start 139.14 79) (end 113.983 79) (width 0.25) (layer F.Cu) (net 5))
 (segment (start 113.983 79) (end 110.873 82.11) (width 0.25) (layer F.Cu) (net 5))
 (segment (start 126.05 82.025) (end 124.174 82.025) (width 0.25) (layer F.Cu) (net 9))
 (segment (start 124.174 82.025) (end 121.294 84.905) (width 0.25) (layer F.Cu) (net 9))
 (segment (start 121.294 84.905) (end 121.294 84.956) (width 0.25) (layer F.Cu) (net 9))
 (segment (start 121.294 84.956) (end 119.25 87) (width 0.25) (layer F.Cu) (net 9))
 (segment (start 126.05 80.075) (end 130.515 80.075) (width 0.25) (layer F.Cu) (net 8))
 (segment (start 135.235 84.905) (end 136.706 84.905) (width 0.25) (layer F.Cu) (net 8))
 (segment (start 135.18 84.96) (end 135.235 84.905) (width 0.25) (layer F.Cu) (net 8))
 (via (at 135.18 84.96) (size 0.6) (drill 0.4) (layers F.Cu B.Cu) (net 8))
 (segment (start 135.18 84.58) (end 135.18 84.96) (width 0.25) (layer B.Cu) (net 8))
 (segment (start 134.9 84.3) (end 135.18 84.58) (width 0.25) (layer B.Cu) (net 8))
 (segment (start 134.9 81.23) (end 134.9 84.3) (width 0.25) (layer B.Cu) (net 8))
 (segment (start 134.9 80.07) (end 134.9 81.23) (width 0.25) (layer B.Cu) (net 8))
 (segment (start 130.52 80.07) (end 134.9 80.07) (width 0.25) (layer B.Cu) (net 8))
 (via (at 130.52 80.07) (size 0.6) (drill 0.4) (layers F.Cu B.Cu) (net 8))
 (segment (start 130.515 80.075) (end 130.52 80.07) (width 0.25) (layer F.Cu) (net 8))
 (segment (start 136.706 84.905) (end 136.706 84.956) (width 0.25) (layer F.Cu) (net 8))
 (segment (start 136.706 84.956) (end 138.75 87) (width 0.25) (layer F.Cu) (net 8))
 (segment (start 131.91 90.95) (end 131.91 89.05) (width 0.25) (layer B.Cu) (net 1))
 (segment (start 131.91 89.05) (end 130.4 89.05) (width 0.25) (layer F.Cu) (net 1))
 (via (at 131.91 89.05) (size 0.6) (drill 0.4) (layers F.Cu B.Cu) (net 1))
 (via (at 131.91 90.95) (size 0.6) (drill 0.4) (layers F.Cu B.Cu) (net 1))
 (segment (start 130.25 96.3) (end 130.25 92.61) (width 0.25) (layer B.Cu) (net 1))
 (segment (start 130.25 92.61) (end 131.91 90.95) (width 0.25) (layer B.Cu) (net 1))
 (segment (start 133.5 90.75) (end 133.75 90.75) (width 0.25) (layer F.Cu) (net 1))
 (segment (start 130.4 90.95) (end 131.91 90.95) (width 0.25) (layer F.Cu) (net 1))
 (segment (start 131.91 90.95) (end 133.3 90.95) (width 0.25) (layer F.Cu) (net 1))
 (segment (start 133.3 90.95) (end 133.5 90.75) (width 0.25) (layer F.Cu) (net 1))
 (segment (start 117.873 98.52) (end 119.4 98.52) (width 0.25) (layer F.Cu) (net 7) (status 400000))
 (segment (start 138.83 91.75) (end 137 91.75) (width 0.25) (layer B.Cu) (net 7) (status 800000))
 (segment (start 139.6 92.52) (end 138.83 91.75) (width 0.25) (layer B.Cu) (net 7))
 (via (at 139.6 92.52) (size 0.6) (drill 0.4) (layers F.Cu B.Cu) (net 7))
 (segment (start 125.4 92.52) (end 139.6 92.52) (width 0.25) (layer F.Cu) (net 7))
 (segment (start 119.4 98.52) (end 125.4 92.52) (width 0.25) (layer F.Cu) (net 7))
 (segment (start 126.05 85.275) (end 129.105 85.275) (width 0.25) (layer F.Cu) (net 7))
 (segment (start 135.42 91.75) (end 137 91.75) (width 0.25) (layer B.Cu) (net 7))
 (segment (start 134.87 91.2) (end 135.42 91.75) (width 0.25) (layer B.Cu) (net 7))
 (segment (start 134.87 87.13) (end 134.87 91.2) (width 0.25) (layer B.Cu) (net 7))
 (via (at 134.87 87.13) (size 0.6) (drill 0.4) (layers F.Cu B.Cu) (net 7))
 (segment (start 130.96 87.13) (end 134.87 87.13) (width 0.25) (layer F.Cu) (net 7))
 (segment (start 129.105 85.275) (end 130.96 87.13) (width 0.25) (layer F.Cu) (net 7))
 (segment (start 127.75 99.5) (end 127.75 98.94) (width 0.25) (layer B.Cu) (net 3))
 (segment (start 127.75 98.94) (end 125.56 96.75) (width 0.25) (layer B.Cu) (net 3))
 (segment (start 125.56 96.75) (end 125.56 87.59) (width 0.25) (layer B.Cu) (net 3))
 (segment (start 125.56 87.59) (end 129.11 84.04) (width 0.25) (layer B.Cu) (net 3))
 (segment (start 129.11 84.04) (end 129.11 80.97) (width 0.25) (layer B.Cu) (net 3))
 (via (at 129.11 80.97) (size 0.6) (drill 0.4) (layers F.Cu B.Cu) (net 3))
 (segment (start 129.11 80.97) (end 130.48 80.97) (width 0.25) (layer F.Cu) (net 3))
 (segment (start 130.48 80.97) (end 130.885 81.375) (width 0.25) (layer F.Cu) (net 3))
 (segment (start 130.885 81.375) (end 131.95 81.375) (width 0.25) (layer F.Cu) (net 3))
 (segment (start 127.75 96.3) (end 127.75 94.16) (width 0.25) (layer B.Cu) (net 2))
 (segment (start 130.075 82.025) (end 131.95 82.025) (width 0.25) (layer F.Cu) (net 2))
 (segment (start 129.97 81.92) (end 130.075 82.025) (width 0.25) (layer F.Cu) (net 2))
 (via (at 129.97 81.92) (size 0.6) (drill 0.4) (layers F.Cu B.Cu) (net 2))
 (segment (start 129.97 84.56) (end 129.97 81.92) (width 0.25) (layer B.Cu) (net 2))
 (segment (start 126.33 88.2) (end 129.97 84.56) (width 0.25) (layer B.Cu) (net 2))
 (segment (start 126.33 92.74) (end 126.33 88.2) (width 0.25) (layer B.Cu) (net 2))
 (segment (start 127.75 94.16) (end 126.33 92.74) (width 0.25) (layer B.Cu) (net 2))
 (segment (start 127.75 96.3) (end 127.75 95.79) (width 0.25) (layer B.Cu) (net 2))
 (segment (start 118.127 95.98) (end 112.297 95.98) (width 0.25) (layer F.Cu) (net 6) (status 400000))
 (segment (start 112.297 95.98) (end 111.127 94.81) (width 0.25) (layer F.Cu) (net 6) (status 800000))
 (segment (start 126.05 84.625) (end 123.615 84.625) (width 0.25) (layer F.Cu) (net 6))
 (segment (start 116.937 89) (end 111.127 94.81) (width 0.25) (layer F.Cu) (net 6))
 (segment (start 119.24 89) (end 116.937 89) (width 0.25) (layer F.Cu) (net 6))
 (segment (start 123.615 84.625) (end 119.24 89) (width 0.25) (layer F.Cu) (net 6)))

